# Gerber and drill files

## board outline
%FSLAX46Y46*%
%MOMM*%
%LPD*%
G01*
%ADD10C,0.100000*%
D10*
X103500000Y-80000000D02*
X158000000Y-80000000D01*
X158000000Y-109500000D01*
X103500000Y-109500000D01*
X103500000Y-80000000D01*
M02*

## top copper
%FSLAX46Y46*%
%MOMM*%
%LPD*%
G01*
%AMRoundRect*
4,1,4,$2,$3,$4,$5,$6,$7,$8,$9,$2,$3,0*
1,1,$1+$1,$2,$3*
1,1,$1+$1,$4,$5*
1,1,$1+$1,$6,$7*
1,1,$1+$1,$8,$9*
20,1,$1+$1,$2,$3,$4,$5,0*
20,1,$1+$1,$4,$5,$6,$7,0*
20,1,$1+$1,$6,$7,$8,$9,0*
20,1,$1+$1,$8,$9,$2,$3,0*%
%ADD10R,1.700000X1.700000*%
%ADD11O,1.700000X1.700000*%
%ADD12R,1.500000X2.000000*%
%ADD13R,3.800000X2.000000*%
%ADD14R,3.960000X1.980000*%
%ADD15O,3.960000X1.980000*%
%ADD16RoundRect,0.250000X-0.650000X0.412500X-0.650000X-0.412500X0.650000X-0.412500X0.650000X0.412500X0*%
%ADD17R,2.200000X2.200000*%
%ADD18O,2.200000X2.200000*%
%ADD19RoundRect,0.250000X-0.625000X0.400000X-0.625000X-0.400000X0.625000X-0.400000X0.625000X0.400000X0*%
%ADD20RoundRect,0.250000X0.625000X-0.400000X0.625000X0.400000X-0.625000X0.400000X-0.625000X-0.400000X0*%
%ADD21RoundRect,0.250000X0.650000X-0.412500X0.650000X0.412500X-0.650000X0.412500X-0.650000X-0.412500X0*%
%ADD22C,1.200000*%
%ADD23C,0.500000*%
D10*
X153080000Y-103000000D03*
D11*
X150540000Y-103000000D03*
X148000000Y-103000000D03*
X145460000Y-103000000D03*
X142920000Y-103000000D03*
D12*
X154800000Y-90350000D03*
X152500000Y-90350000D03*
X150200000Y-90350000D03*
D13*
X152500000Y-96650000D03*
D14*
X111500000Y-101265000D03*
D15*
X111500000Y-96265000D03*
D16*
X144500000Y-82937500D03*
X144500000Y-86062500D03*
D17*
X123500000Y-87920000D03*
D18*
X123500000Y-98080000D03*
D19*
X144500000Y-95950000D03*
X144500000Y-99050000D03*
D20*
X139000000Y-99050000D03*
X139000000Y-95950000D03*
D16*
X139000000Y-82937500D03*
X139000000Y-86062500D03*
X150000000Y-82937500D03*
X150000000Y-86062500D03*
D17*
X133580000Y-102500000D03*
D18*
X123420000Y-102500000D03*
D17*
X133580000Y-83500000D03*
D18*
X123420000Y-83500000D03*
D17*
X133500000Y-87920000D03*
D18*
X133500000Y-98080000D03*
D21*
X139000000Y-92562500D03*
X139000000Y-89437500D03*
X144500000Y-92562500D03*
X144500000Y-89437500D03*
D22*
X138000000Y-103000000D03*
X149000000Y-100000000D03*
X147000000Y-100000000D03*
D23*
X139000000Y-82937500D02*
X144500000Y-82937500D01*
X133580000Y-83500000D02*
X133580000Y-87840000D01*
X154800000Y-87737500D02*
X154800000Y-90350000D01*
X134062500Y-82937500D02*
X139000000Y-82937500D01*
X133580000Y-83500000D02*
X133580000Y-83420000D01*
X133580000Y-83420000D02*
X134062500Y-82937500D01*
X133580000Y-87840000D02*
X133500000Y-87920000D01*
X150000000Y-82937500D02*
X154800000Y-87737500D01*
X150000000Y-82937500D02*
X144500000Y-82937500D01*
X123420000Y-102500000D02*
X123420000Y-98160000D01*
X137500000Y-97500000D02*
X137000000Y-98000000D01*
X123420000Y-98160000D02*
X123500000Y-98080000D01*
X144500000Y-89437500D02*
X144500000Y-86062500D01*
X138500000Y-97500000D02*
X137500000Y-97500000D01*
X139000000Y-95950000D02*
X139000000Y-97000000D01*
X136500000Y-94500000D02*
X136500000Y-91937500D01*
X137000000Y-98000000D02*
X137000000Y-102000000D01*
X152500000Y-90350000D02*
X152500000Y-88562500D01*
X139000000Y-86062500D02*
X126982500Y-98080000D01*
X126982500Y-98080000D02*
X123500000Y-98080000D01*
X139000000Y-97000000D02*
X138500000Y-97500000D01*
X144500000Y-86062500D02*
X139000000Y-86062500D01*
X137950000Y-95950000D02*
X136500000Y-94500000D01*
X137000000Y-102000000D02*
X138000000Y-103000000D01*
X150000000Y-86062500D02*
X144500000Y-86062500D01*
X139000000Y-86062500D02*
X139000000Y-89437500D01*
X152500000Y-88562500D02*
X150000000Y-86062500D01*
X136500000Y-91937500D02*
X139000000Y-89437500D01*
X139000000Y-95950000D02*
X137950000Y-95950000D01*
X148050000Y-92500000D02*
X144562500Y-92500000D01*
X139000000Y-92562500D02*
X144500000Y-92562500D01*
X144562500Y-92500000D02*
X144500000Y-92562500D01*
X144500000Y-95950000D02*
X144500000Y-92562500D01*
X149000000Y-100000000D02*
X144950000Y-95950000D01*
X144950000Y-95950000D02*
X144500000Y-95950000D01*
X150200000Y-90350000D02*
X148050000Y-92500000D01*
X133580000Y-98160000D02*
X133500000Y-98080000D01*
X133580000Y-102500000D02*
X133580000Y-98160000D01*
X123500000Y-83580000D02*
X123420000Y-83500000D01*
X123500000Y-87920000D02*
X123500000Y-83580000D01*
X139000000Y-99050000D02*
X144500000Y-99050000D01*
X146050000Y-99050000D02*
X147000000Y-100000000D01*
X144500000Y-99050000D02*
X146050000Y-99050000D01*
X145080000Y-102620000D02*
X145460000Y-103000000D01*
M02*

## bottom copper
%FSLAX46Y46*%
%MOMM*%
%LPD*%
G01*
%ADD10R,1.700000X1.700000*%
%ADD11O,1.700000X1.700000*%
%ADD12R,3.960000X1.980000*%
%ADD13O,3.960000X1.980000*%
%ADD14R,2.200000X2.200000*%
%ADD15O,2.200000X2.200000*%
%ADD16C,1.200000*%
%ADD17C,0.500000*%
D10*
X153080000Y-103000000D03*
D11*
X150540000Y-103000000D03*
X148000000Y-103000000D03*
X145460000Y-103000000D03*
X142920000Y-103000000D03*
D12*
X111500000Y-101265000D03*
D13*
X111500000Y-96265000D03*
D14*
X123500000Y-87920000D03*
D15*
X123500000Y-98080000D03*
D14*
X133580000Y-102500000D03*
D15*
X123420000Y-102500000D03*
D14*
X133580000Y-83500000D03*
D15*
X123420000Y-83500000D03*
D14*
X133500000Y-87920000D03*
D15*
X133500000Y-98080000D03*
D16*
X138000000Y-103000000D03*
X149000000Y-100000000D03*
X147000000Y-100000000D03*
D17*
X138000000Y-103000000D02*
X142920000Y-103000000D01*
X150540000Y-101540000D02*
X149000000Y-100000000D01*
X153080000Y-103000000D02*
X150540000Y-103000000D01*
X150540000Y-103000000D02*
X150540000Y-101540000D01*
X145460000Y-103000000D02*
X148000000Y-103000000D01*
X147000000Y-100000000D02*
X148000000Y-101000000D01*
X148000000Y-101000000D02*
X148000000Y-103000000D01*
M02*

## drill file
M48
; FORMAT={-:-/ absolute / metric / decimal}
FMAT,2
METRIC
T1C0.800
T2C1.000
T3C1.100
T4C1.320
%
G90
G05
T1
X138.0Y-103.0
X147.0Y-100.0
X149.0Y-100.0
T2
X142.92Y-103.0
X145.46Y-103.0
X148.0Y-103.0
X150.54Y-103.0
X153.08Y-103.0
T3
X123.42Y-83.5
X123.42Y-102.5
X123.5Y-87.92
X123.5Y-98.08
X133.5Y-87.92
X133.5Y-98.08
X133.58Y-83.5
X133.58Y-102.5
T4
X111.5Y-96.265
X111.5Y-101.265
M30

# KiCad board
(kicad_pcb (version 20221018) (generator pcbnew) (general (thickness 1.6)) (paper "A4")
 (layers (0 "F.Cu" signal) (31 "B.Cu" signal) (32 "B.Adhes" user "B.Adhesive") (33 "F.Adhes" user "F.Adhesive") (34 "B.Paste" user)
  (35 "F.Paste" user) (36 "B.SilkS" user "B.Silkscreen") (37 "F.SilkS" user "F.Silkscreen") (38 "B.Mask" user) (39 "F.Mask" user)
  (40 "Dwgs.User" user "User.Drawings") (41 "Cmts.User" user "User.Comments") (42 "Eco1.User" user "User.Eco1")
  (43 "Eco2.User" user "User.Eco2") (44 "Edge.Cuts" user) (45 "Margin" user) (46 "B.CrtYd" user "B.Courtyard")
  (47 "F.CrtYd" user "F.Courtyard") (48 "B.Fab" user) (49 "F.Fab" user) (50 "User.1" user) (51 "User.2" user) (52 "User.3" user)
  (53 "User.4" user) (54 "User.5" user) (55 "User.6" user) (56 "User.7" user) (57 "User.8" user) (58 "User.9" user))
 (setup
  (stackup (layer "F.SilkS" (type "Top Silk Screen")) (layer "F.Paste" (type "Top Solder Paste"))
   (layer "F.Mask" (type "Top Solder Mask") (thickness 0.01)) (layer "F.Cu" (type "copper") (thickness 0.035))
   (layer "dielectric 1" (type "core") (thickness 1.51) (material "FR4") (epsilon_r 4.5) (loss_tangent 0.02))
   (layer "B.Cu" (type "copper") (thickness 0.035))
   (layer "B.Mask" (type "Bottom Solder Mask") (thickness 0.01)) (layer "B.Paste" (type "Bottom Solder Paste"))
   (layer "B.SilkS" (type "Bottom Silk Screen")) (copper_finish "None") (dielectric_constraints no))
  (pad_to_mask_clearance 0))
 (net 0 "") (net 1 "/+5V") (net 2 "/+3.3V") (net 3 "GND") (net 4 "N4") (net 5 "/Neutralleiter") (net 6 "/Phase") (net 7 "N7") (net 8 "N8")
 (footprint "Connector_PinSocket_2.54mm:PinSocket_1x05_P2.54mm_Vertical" (layer "F.Cu") (at 153.08 103 -90)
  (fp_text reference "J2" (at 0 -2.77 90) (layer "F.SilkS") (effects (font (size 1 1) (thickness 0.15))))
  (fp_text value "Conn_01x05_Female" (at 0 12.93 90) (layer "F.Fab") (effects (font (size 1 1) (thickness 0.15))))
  (pad "1" thru_hole rect (at 0 0 270) (size 1.7 1.7) (drill 1) (layers "*.Cu" "*.Mask") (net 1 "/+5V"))
  (pad "2" thru_hole oval (at 0 2.54 270) (size 1.7 1.7) (drill 1) (layers "*.Cu" "*.Mask") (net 1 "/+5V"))
  (pad "3" thru_hole oval (at 0 5.08 270) (size 1.7 1.7) (drill 1) (layers "*.Cu" "*.Mask") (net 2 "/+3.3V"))
  (pad "4" thru_hole oval (at 0 7.62 270) (size 1.7 1.7) (drill 1) (layers "*.Cu" "*.Mask") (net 2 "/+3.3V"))
  (pad "5" thru_hole oval (at 0 10.16 270) (size 1.7 1.7) (drill 1) (layers "*.Cu" "*.Mask") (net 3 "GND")))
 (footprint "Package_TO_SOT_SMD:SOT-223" (layer "F.Cu") (at 152.5 93.5 -90)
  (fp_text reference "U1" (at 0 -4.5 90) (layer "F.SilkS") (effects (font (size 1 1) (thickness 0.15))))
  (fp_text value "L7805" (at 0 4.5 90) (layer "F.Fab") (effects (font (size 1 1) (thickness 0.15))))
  (pad "1" smd rect (at -3.15 -2.3 270) (size 2 1.5) (layers "F.Cu" "F.Paste" "F.Mask") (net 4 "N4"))
  (pad "2" smd rect (at -3.15 0 270) (size 2 1.5) (layers "F.Cu" "F.Paste" "F.Mask") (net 3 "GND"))
  (pad "3" smd rect (at -3.15 2.3 270) (size 2 1.5) (layers "F.Cu" "F.Paste" "F.Mask") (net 1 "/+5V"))
  (pad "4" smd rect (at 3.15 0 270) (size 2 3.8) (layers "F.Cu" "F.Paste" "F.Mask")))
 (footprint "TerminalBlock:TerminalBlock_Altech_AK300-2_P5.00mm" (layer "F.Cu") (at 111.5 101.265 90)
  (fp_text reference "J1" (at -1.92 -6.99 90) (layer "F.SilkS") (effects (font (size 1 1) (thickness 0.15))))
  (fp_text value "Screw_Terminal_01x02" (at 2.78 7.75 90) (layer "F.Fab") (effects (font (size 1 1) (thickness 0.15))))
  (pad "1" thru_hole rect (at 0 0 90) (size 1.98 3.96) (drill 1.32) (layers "*.Cu" "*.Mask") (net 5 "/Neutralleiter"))
  (pad "2" thru_hole oval (at 5 0 90) (size 1.98 3.96) (drill 1.32) (layers "*.Cu" "*.Mask") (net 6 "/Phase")))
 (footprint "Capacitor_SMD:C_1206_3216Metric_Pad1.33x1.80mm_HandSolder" (layer "F.Cu") (at 144.5 84.5 -90)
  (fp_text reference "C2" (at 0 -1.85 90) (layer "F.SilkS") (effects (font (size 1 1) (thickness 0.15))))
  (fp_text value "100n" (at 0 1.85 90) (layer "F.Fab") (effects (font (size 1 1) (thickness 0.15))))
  (pad "1" smd roundrect (at -1.5625 0 270) (size 1.325 1.8) (layers "F.Cu" "F.Paste" "F.Mask") (roundrect_rratio 0.188679) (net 4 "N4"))
  (pad "2" smd roundrect (at 1.5625 0 270) (size 1.325 1.8) (layers "F.Cu" "F.Paste" "F.Mask") (roundrect_rratio 0.188679) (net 3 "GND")))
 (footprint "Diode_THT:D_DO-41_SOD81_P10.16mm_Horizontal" (layer "F.Cu") (at 123.5 87.92 -90)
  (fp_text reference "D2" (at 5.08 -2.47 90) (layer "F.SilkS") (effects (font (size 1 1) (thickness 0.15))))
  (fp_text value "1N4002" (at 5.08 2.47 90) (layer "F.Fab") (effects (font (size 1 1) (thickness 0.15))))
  (pad "1" thru_hole rect (at 0 0 270) (size 2.2 2.2) (drill 1.1) (layers "*.Cu" "*.Mask") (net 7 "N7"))
  (pad "2" thru_hole oval (at 10.16 0 270) (size 2.2 2.2) (drill 1.1) (layers "*.Cu" "*.Mask") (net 3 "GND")))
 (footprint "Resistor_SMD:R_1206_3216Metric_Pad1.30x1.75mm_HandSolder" (layer "F.Cu") (at 144.5 97.5 -90)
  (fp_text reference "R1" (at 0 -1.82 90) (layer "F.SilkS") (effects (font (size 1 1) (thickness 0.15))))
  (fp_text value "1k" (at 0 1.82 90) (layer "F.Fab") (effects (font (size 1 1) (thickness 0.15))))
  (pad "1" smd roundrect (at -1.55 0 270) (size 1.3 1.75) (layers "F.Cu" "F.Paste" "F.Mask") (roundrect_rratio 0.192308) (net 1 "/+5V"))
  (pad "2" smd roundrect (at 1.55 0 270) (size 1.3 1.75) (layers "F.Cu" "F.Paste" "F.Mask") (roundrect_rratio 0.192308) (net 2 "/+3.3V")))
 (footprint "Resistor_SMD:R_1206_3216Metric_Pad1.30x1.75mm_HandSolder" (layer "F.Cu") (at 139 97.5 90)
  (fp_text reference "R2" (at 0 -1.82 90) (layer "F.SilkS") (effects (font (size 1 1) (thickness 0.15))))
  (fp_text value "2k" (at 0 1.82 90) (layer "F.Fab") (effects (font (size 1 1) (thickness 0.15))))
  (pad "1" smd roundrect (at -1.55 0 90) (size 1.3 1.75) (layers "F.Cu" "F.Paste" "F.Mask") (roundrect_rratio 0.192308) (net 2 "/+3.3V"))
  (pad "2" smd roundrect (at 1.55 0 90) (size 1.3 1.75) (layers "F.Cu" "F.Paste" "F.Mask") (roundrect_rratio 0.192308) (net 3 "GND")))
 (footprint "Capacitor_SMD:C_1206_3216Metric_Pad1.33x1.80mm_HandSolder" (layer "F.Cu") (at 139 84.5 -90)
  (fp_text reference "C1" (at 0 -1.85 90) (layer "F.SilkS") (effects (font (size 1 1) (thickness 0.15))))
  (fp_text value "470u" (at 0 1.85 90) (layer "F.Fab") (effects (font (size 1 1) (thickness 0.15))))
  (pad "1" smd roundrect (at -1.5625 0 270) (size 1.325 1.8) (layers "F.Cu" "F.Paste" "F.Mask") (roundrect_rratio 0.188679) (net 4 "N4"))
  (pad "2" smd roundrect (at 1.5625 0 270) (size 1.325 1.8) (layers "F.Cu" "F.Paste" "F.Mask") (roundrect_rratio 0.188679) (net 3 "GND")))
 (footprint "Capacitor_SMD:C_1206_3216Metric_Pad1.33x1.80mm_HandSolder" (layer "F.Cu") (at 150 84.5 -90)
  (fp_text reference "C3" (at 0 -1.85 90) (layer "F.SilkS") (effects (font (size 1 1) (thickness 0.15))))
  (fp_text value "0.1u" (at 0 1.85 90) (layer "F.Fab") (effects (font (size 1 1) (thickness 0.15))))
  (pad "1" smd roundrect (at -1.5625 0 270) (size 1.325 1.8) (layers "F.Cu" "F.Paste" "F.Mask") (roundrect_rratio 0.188679) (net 4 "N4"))
  (pad "2" smd roundrect (at 1.5625 0 270) (size 1.325 1.8) (layers "F.Cu" "F.Paste" "F.Mask") (roundrect_rratio 0.188679) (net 3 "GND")))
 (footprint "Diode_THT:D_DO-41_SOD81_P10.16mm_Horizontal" (layer "F.Cu") (at 133.58 102.5 180)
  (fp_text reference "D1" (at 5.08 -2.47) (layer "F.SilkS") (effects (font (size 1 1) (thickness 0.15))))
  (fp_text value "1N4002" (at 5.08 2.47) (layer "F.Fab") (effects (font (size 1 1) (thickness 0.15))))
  (pad "1" thru_hole rect (at 0 0 180) (size 2.2 2.2) (drill 1.1) (layers "*.Cu" "*.Mask") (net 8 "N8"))
  (pad "2" thru_hole oval (at 10.16 0 180) (size 2.2 2.2) (drill 1.1) (layers "*.Cu" "*.Mask") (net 3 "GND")))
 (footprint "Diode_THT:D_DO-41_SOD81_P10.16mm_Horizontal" (layer "F.Cu") (at 133.58 83.5 180)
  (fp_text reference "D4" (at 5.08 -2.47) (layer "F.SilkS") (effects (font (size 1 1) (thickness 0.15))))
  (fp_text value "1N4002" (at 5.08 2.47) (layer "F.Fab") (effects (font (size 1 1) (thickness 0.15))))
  (pad "1" thru_hole rect (at 0 0 180) (size 2.2 2.2) (drill 1.1) (layers "*.Cu" "*.Mask") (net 4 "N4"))
  (pad "2" thru_hole oval (at 10.16 0 180) (size 2.2 2.2) (drill 1.1) (layers "*.Cu" "*.Mask") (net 7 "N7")))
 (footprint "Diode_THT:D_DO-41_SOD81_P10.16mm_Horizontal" (layer "F.Cu") (at 133.5 87.92 -90)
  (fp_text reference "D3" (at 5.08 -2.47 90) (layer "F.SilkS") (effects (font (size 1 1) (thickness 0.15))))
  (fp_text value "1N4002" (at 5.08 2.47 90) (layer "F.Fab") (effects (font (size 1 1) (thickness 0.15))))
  (pad "1" thru_hole rect (at 0 0 270) (size 2.2 2.2) (drill 1.1) (layers "*.Cu" "*.Mask") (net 4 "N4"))
  (pad "2" thru_hole oval (at 10.16 0 270) (size 2.2 2.2) (drill 1.1) (layers "*.Cu" "*.Mask") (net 8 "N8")))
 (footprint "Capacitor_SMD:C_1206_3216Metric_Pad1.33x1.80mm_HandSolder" (layer "F.Cu") (at 139 91 90)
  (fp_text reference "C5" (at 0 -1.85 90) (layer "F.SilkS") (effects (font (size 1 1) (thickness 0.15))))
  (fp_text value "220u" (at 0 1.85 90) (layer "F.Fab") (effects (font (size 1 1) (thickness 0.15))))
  (pad "1" smd roundrect (at -1.5625 0 90) (size 1.325 1.8) (layers "F.Cu" "F.Paste" "F.Mask") (roundrect_rratio 0.188679) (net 1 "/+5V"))
  (pad "2" smd roundrect (at 1.5625 0 90) (size 1.325 1.8) (layers "F.Cu" "F.Paste" "F.Mask") (roundrect_rratio 0.188679) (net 3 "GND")))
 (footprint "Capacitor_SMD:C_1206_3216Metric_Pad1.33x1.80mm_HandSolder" (layer "F.Cu") (at 144.5 91 90)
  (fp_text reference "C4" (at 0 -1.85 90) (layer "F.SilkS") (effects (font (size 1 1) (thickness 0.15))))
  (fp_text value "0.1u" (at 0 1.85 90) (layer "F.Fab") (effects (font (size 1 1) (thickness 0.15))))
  (pad "1" smd roundrect (at -1.5625 0 90) (size 1.325 1.8) (layers "F.Cu" "F.Paste" "F.Mask") (roundrect_rratio 0.188679) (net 1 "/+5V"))
  (pad "2" smd roundrect (at 1.5625 0 90) (size 1.325 1.8) (layers "F.Cu" "F.Paste" "F.Mask") (roundrect_rratio 0.188679) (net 3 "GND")))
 (gr_rect (start 103.5 80) (end 158 109.5) (stroke (width 0.1) (type solid)) (fill none) (layer "Edge.Cuts"))
 (segment (start 139 82.9375) (end 144.5 82.9375) (width 0.5) (layer "F.Cu") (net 4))
 (segment (start 133.58 83.5) (end 133.58 87.84) (width 0.5) (layer "F.Cu") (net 4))
 (segment (start 154.8 87.7375) (end 154.8 90.35) (width 0.5) (layer "F.Cu") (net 4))
 (segment (start 134.0625 82.9375) (end 139 82.9375) (width 0.5) (layer "F.Cu") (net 4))
 (segment (start 133.58 83.5) (end 133.58 83.42) (width 0.5) (layer "F.Cu") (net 4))
 (segment (start 133.58 83.42) (end 134.0625 82.9375) (width 0.5) (layer "F.Cu") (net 4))
 (segment (start 133.58 87.84) (end 133.5 87.92) (width 0.5) (layer "F.Cu") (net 4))
 (segment (start 150 82.9375) (end 154.8 87.7375) (width 0.5) (layer "F.Cu") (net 4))
 (segment (start 150 82.9375) (end 144.5 82.9375) (width 0.5) (layer "F.Cu") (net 4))
 (segment (start 123.42 102.5) (end 123.42 98.16) (width 0.5) (layer "F.Cu") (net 3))
 (segment (start 137.5 97.5) (end 137 98) (width 0.5) (layer "F.Cu") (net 3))
 (segment (start 123.42 98.16) (end 123.5 98.08) (width 0.5) (layer "F.Cu") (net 3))
 (segment (start 144.5 89.4375) (end 144.5 86.0625) (width 0.5) (layer "F.Cu") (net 3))
 (segment (start 138.5 97.5) (end 137.5 97.5) (width 0.5) (layer "F.Cu") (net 3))
 (segment (start 139 95.95) (end 139 97) (width 0.5) (layer "F.Cu") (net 3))
 (segment (start 136.5 94.5) (end 136.5 91.9375) (width 0.5) (layer "F.Cu") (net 3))
 (segment (start 137 98) (end 137 102) (width 0.5) (layer "F.Cu") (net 3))
 (segment (start 152.5 90.35) (end 152.5 88.5625) (width 0.5) (layer "F.Cu") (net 3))
 (segment (start 139 86.0625) (end 126.9825 98.08) (width 0.5) (layer "F.Cu") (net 3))
 (segment (start 126.9825 98.08) (end 123.5 98.08) (width 0.5) (layer "F.Cu") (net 3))
 (segment (start 139 97) (end 138.5 97.5) (width 0.5) (layer "F.Cu") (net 3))
 (segment (start 144.5 86.0625) (end 139 86.0625) (width 0.5) (layer "F.Cu") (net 3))
 (segment (start 137.95 95.95) (end 136.5 94.5) (width 0.5) (layer "F.Cu") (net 3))
 (segment (start 137 102) (end 138 103) (width 0.5) (layer "F.Cu") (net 3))
 (segment (start 150 86.0625) (end 144.5 86.0625) (width 0.5) (layer "F.Cu") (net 3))
 (segment (start 139 86.0625) (end 139 89.4375) (width 0.5) (layer "F.Cu") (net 3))
 (segment (start 152.5 88.5625) (end 150 86.0625) (width 0.5) (layer "F.Cu") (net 3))
 (segment (start 136.5 91.9375) (end 139 89.4375) (width 0.5) (layer "F.Cu") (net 3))
 (segment (start 139 95.95) (end 137.95 95.95) (width 0.5) (layer "F.Cu") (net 3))
 (via (at 138 103) (size 1.2) (drill 0.8) (layers "F.Cu" "B.Cu") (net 3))
 (segment (start 138 103) (end 142.92 103) (width 0.5) (layer "B.Cu") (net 3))
 (segment (start 148.05 92.5) (end 144.5625 92.5) (width 0.5) (layer "F.Cu") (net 1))
 (segment (start 139 92.5625) (end 144.5 92.5625) (width 0.5) (layer "F.Cu") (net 1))
 (segment (start 144.5625 92.5) (end 144.5 92.5625) (width 0.5) (layer "F.Cu") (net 1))
 (segment (start 144.5 95.95) (end 144.5 92.5625) (width 0.5) (layer "F.Cu") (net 1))
 (segment (start 149 100) (end 144.95 95.95) (width 0.5) (layer "F.Cu") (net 1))
 (segment (start 144.95 95.95) (end 144.5 95.95) (width 0.5) (layer "F.Cu") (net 1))
 (segment (start 150.2 90.35) (end 148.05 92.5) (width 0.5) (layer "F.Cu") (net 1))
 (via (at 149 100) (size 1.2) (drill 0.8) (layers "F.Cu" "B.Cu") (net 1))
 (segment (start 150.54 101.54) (end 149 100) (width 0.5) (layer "B.Cu") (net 1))
 (segment (start 153.08 103) (end 150.54 103) (width 0.5) (layer "B.Cu") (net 1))
 (segment (start 150.54 103) (end 150.54 101.54) (width 0.5) (layer "B.Cu") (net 1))
 (segment (start 133.58 98.16) (end 133.5 98.08) (width 0.5) (layer "F.Cu") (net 8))
 (segment (start 133.58 102.5) (end 133.58 98.16) (width 0.5) (layer "F.Cu") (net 8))
 (segment (start 123.5 83.58) (end 123.42 83.5) (width 0.5) (layer "F.Cu") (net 7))
 (segment (start 123.5 87.92) (end 123.5 83.58) (width 0.5) (layer "F.Cu") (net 7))
 (segment (start 139 99.05) (end 144.5 99.05) (width 0.5) (layer "F.Cu") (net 2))
 (segment (start 146.05 99.05) (end 147 100) (width 0.5) (layer "F.Cu") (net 2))
 (segment (start 144.5 99.05) (end 146.05 99.05) (width 0.5) (layer "F.Cu") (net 2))
 (segment (start 145.08 102.62) (end 145.46 103) (width 0.5) (layer "F.Cu") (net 2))
 (via (at 147 100) (size 1.2) (drill 0.8) (layers "F.Cu" "B.Cu") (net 2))
 (segment (start 145.46 103) (end 148 103) (width 0.5) (layer "B.Cu") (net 2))
 (segment (start 147 100) (end 148 101) (width 0.5) (layer "B.Cu") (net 2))
 (segment (start 148 101) (end 148 103) (width 0.5) (layer "B.Cu") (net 2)))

